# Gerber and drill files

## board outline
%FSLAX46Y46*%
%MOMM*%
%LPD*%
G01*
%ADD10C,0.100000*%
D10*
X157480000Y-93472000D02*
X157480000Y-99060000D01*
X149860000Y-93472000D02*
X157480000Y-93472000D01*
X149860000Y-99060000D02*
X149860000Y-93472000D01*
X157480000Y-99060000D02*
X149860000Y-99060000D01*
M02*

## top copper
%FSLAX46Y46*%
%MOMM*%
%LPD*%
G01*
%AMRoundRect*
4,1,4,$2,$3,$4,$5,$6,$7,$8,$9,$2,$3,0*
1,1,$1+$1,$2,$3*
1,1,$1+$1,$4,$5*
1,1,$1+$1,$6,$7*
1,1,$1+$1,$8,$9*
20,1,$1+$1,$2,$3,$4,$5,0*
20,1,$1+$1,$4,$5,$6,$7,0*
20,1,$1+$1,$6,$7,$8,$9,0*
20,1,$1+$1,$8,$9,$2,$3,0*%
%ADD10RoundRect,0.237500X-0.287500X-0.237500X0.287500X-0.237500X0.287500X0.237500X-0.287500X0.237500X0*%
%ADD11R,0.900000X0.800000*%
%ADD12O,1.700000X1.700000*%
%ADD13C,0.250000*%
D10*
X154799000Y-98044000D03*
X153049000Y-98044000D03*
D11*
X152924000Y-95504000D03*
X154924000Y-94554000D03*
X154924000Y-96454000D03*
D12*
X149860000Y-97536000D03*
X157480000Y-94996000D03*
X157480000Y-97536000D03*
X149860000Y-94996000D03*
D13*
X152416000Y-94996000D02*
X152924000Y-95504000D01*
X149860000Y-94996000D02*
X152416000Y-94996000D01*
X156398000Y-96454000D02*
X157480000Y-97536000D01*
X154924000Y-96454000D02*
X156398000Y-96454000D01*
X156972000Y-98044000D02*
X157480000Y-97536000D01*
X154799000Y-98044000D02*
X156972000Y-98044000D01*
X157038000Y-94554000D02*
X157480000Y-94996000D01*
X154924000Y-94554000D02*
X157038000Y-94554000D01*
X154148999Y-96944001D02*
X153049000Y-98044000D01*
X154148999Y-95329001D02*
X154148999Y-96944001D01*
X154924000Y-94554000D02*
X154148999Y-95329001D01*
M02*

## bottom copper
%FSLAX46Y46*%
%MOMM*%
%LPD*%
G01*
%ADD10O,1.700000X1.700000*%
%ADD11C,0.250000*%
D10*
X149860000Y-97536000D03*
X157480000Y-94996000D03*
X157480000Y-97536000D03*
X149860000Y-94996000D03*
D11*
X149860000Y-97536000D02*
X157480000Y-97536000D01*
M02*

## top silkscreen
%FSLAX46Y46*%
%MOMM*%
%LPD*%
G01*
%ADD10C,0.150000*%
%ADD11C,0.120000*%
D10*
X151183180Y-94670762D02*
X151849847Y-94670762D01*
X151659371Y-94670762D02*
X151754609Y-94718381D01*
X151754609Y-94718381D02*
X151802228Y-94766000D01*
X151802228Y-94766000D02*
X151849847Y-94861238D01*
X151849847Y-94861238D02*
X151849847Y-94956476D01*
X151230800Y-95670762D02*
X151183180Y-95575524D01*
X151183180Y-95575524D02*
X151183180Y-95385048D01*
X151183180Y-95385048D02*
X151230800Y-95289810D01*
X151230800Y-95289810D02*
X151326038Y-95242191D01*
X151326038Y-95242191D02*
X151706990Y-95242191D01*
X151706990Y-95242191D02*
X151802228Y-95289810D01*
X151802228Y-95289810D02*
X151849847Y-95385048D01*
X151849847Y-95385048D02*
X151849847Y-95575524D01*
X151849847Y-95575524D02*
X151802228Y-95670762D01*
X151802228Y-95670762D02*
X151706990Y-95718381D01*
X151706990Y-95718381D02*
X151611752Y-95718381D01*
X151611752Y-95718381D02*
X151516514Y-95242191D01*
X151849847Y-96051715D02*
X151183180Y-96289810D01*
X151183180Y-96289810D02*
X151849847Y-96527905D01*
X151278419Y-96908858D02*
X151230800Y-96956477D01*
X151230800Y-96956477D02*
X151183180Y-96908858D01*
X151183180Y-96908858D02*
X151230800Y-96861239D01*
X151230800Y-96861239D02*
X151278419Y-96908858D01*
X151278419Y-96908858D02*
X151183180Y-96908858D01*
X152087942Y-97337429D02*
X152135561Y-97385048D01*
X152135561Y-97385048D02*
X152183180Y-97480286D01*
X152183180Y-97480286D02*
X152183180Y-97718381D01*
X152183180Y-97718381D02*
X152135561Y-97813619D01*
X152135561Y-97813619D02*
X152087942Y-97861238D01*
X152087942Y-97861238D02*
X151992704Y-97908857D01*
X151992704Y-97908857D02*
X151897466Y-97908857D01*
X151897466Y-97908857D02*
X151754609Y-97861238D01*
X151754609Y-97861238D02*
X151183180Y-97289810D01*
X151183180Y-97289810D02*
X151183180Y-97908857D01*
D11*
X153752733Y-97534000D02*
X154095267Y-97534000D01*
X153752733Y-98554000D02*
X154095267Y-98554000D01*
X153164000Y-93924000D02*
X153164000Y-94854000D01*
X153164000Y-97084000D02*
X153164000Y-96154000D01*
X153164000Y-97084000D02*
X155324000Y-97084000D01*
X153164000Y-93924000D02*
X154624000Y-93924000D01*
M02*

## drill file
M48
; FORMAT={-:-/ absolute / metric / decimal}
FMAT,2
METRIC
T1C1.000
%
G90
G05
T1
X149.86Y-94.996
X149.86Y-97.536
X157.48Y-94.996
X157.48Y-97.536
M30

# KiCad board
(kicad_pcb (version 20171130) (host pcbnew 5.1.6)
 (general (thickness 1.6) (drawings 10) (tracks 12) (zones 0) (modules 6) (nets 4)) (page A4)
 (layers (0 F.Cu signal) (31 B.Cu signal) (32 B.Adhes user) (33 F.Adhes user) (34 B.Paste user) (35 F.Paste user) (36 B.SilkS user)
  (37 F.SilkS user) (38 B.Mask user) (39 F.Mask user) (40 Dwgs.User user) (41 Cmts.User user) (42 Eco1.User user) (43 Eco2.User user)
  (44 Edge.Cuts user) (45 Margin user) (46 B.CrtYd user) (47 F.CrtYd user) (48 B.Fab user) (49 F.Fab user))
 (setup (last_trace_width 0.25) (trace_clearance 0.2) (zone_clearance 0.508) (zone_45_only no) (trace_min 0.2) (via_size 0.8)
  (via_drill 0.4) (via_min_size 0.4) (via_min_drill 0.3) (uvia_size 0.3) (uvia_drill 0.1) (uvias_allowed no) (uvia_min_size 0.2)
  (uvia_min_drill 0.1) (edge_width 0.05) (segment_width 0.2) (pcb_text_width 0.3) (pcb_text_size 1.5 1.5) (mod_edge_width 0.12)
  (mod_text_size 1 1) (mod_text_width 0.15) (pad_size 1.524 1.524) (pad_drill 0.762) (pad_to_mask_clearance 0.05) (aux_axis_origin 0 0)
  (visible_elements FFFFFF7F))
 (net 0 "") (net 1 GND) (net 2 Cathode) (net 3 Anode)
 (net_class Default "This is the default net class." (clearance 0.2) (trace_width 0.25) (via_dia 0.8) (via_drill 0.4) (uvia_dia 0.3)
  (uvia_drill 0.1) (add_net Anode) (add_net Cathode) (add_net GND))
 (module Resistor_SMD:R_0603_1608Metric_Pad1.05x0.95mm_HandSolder (layer F.Cu) (at 153.924 98.044)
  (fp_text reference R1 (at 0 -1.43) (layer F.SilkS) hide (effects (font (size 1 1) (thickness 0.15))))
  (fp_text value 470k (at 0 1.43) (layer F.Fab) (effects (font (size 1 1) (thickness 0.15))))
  (fp_line (start -0.171267 -0.51) (end 0.171267 -0.51) (layer F.SilkS) (width 0.12))
  (fp_line (start -0.171267 0.51) (end 0.171267 0.51) (layer F.SilkS) (width 0.12))
  (pad 2 smd roundrect (at 0.875 0) (size 1.05 0.95) (layers F.Cu F.Paste F.Mask) (roundrect_rratio 0.25) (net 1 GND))
  (pad 1 smd roundrect (at -0.875 0) (size 1.05 0.95) (layers F.Cu F.Paste F.Mask) (roundrect_rratio 0.25) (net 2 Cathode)))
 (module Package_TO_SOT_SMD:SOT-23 (layer F.Cu) (at 153.924 95.504 180)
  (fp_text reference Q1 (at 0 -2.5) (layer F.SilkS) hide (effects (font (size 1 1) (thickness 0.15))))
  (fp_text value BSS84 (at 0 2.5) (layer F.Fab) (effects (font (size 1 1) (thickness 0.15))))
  (fp_line (start 0.76 1.58) (end 0.76 0.65) (layer F.SilkS) (width 0.12))
  (fp_line (start 0.76 -1.58) (end 0.76 -0.65) (layer F.SilkS) (width 0.12))
  (fp_line (start 0.76 -1.58) (end -1.4 -1.58) (layer F.SilkS) (width 0.12))
  (fp_line (start 0.76 1.58) (end -0.7 1.58) (layer F.SilkS) (width 0.12))
  (pad 3 smd rect (at 1 0 180) (size 0.9 0.8) (layers F.Cu F.Paste F.Mask) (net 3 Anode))
  (pad 2 smd rect (at -1 0.95 180) (size 0.9 0.8) (layers F.Cu F.Paste F.Mask) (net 2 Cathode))
  (pad 1 smd rect (at -1 -0.95 180) (size 0.9 0.8) (layers F.Cu F.Paste F.Mask) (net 1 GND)))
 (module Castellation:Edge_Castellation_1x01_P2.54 (layer F.Cu) (at 149.86 97.536)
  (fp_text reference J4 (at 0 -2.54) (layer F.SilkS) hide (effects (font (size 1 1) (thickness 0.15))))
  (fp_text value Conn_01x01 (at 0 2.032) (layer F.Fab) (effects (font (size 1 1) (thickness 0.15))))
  (pad 1 thru_hole oval (at 0 0) (size 1.7 1.7) (drill 1) (layers *.Cu *.Mask) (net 1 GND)))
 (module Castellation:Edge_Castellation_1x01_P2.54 (layer F.Cu) (at 157.48 94.996)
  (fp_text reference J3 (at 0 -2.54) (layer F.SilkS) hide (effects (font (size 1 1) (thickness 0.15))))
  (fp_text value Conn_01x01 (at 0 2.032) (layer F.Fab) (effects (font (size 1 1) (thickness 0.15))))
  (pad 1 thru_hole oval (at 0 0) (size 1.7 1.7) (drill 1) (layers *.Cu *.Mask) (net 2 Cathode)))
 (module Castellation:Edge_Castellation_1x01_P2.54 (layer F.Cu) (at 157.48 97.536)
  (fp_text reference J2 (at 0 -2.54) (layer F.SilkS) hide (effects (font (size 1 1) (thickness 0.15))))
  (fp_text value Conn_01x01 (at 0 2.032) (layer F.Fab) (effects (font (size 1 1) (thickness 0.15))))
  (pad 1 thru_hole oval (at 0 0) (size 1.7 1.7) (drill 1) (layers *.Cu *.Mask) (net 1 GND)))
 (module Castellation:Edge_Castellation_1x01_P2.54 (layer F.Cu) (at 149.86 94.996)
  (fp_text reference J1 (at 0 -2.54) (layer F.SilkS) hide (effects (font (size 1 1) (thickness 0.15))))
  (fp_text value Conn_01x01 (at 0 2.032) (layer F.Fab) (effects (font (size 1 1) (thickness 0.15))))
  (pad 1 thru_hole oval (at 0 0) (size 1.7 1.7) (drill 1) (layers *.Cu *.Mask) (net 3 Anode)))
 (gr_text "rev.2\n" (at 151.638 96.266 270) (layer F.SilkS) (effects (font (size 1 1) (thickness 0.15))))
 (gr_line (start 157.48 93.472) (end 157.48 99.06) (layer Edge.Cuts) (width 0.1))
 (gr_line (start 149.86 93.472) (end 157.48 93.472) (layer Edge.Cuts) (width 0.1))
 (gr_line (start 149.86 99.06) (end 149.86 93.472) (layer Edge.Cuts) (width 0.1))
 (gr_line (start 157.48 99.06) (end 149.86 99.06) (layer Edge.Cuts) (width 0.1))
 (segment (start 152.416 94.996) (end 152.924 95.504) (width 0.25) (layer F.Cu) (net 3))
 (segment (start 149.86 94.996) (end 152.416 94.996) (width 0.25) (layer F.Cu) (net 3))
 (segment (start 156.398 96.454) (end 157.48 97.536) (width 0.25) (layer F.Cu) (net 1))
 (segment (start 154.924 96.454) (end 156.398 96.454) (width 0.25) (layer F.Cu) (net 1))
 (segment (start 156.972 98.044) (end 157.48 97.536) (width 0.25) (layer F.Cu) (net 1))
 (segment (start 154.799 98.044) (end 156.972 98.044) (width 0.25) (layer F.Cu) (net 1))
 (segment (start 149.86 97.536) (end 157.48 97.536) (width 0.25) (layer B.Cu) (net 1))
 (segment (start 157.038 94.554) (end 157.48 94.996) (width 0.25) (layer F.Cu) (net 2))
 (segment (start 154.924 94.554) (end 157.038 94.554) (width 0.25) (layer F.Cu) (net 2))
 (segment (start 154.148999 96.944001) (end 153.049 98.044) (width 0.25) (layer F.Cu) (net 2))
 (segment (start 154.148999 95.329001) (end 154.148999 96.944001) (width 0.25) (layer F.Cu) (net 2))
 (segment (start 154.924 94.554) (end 154.148999 95.329001) (width 0.25) (layer F.Cu) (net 2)))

